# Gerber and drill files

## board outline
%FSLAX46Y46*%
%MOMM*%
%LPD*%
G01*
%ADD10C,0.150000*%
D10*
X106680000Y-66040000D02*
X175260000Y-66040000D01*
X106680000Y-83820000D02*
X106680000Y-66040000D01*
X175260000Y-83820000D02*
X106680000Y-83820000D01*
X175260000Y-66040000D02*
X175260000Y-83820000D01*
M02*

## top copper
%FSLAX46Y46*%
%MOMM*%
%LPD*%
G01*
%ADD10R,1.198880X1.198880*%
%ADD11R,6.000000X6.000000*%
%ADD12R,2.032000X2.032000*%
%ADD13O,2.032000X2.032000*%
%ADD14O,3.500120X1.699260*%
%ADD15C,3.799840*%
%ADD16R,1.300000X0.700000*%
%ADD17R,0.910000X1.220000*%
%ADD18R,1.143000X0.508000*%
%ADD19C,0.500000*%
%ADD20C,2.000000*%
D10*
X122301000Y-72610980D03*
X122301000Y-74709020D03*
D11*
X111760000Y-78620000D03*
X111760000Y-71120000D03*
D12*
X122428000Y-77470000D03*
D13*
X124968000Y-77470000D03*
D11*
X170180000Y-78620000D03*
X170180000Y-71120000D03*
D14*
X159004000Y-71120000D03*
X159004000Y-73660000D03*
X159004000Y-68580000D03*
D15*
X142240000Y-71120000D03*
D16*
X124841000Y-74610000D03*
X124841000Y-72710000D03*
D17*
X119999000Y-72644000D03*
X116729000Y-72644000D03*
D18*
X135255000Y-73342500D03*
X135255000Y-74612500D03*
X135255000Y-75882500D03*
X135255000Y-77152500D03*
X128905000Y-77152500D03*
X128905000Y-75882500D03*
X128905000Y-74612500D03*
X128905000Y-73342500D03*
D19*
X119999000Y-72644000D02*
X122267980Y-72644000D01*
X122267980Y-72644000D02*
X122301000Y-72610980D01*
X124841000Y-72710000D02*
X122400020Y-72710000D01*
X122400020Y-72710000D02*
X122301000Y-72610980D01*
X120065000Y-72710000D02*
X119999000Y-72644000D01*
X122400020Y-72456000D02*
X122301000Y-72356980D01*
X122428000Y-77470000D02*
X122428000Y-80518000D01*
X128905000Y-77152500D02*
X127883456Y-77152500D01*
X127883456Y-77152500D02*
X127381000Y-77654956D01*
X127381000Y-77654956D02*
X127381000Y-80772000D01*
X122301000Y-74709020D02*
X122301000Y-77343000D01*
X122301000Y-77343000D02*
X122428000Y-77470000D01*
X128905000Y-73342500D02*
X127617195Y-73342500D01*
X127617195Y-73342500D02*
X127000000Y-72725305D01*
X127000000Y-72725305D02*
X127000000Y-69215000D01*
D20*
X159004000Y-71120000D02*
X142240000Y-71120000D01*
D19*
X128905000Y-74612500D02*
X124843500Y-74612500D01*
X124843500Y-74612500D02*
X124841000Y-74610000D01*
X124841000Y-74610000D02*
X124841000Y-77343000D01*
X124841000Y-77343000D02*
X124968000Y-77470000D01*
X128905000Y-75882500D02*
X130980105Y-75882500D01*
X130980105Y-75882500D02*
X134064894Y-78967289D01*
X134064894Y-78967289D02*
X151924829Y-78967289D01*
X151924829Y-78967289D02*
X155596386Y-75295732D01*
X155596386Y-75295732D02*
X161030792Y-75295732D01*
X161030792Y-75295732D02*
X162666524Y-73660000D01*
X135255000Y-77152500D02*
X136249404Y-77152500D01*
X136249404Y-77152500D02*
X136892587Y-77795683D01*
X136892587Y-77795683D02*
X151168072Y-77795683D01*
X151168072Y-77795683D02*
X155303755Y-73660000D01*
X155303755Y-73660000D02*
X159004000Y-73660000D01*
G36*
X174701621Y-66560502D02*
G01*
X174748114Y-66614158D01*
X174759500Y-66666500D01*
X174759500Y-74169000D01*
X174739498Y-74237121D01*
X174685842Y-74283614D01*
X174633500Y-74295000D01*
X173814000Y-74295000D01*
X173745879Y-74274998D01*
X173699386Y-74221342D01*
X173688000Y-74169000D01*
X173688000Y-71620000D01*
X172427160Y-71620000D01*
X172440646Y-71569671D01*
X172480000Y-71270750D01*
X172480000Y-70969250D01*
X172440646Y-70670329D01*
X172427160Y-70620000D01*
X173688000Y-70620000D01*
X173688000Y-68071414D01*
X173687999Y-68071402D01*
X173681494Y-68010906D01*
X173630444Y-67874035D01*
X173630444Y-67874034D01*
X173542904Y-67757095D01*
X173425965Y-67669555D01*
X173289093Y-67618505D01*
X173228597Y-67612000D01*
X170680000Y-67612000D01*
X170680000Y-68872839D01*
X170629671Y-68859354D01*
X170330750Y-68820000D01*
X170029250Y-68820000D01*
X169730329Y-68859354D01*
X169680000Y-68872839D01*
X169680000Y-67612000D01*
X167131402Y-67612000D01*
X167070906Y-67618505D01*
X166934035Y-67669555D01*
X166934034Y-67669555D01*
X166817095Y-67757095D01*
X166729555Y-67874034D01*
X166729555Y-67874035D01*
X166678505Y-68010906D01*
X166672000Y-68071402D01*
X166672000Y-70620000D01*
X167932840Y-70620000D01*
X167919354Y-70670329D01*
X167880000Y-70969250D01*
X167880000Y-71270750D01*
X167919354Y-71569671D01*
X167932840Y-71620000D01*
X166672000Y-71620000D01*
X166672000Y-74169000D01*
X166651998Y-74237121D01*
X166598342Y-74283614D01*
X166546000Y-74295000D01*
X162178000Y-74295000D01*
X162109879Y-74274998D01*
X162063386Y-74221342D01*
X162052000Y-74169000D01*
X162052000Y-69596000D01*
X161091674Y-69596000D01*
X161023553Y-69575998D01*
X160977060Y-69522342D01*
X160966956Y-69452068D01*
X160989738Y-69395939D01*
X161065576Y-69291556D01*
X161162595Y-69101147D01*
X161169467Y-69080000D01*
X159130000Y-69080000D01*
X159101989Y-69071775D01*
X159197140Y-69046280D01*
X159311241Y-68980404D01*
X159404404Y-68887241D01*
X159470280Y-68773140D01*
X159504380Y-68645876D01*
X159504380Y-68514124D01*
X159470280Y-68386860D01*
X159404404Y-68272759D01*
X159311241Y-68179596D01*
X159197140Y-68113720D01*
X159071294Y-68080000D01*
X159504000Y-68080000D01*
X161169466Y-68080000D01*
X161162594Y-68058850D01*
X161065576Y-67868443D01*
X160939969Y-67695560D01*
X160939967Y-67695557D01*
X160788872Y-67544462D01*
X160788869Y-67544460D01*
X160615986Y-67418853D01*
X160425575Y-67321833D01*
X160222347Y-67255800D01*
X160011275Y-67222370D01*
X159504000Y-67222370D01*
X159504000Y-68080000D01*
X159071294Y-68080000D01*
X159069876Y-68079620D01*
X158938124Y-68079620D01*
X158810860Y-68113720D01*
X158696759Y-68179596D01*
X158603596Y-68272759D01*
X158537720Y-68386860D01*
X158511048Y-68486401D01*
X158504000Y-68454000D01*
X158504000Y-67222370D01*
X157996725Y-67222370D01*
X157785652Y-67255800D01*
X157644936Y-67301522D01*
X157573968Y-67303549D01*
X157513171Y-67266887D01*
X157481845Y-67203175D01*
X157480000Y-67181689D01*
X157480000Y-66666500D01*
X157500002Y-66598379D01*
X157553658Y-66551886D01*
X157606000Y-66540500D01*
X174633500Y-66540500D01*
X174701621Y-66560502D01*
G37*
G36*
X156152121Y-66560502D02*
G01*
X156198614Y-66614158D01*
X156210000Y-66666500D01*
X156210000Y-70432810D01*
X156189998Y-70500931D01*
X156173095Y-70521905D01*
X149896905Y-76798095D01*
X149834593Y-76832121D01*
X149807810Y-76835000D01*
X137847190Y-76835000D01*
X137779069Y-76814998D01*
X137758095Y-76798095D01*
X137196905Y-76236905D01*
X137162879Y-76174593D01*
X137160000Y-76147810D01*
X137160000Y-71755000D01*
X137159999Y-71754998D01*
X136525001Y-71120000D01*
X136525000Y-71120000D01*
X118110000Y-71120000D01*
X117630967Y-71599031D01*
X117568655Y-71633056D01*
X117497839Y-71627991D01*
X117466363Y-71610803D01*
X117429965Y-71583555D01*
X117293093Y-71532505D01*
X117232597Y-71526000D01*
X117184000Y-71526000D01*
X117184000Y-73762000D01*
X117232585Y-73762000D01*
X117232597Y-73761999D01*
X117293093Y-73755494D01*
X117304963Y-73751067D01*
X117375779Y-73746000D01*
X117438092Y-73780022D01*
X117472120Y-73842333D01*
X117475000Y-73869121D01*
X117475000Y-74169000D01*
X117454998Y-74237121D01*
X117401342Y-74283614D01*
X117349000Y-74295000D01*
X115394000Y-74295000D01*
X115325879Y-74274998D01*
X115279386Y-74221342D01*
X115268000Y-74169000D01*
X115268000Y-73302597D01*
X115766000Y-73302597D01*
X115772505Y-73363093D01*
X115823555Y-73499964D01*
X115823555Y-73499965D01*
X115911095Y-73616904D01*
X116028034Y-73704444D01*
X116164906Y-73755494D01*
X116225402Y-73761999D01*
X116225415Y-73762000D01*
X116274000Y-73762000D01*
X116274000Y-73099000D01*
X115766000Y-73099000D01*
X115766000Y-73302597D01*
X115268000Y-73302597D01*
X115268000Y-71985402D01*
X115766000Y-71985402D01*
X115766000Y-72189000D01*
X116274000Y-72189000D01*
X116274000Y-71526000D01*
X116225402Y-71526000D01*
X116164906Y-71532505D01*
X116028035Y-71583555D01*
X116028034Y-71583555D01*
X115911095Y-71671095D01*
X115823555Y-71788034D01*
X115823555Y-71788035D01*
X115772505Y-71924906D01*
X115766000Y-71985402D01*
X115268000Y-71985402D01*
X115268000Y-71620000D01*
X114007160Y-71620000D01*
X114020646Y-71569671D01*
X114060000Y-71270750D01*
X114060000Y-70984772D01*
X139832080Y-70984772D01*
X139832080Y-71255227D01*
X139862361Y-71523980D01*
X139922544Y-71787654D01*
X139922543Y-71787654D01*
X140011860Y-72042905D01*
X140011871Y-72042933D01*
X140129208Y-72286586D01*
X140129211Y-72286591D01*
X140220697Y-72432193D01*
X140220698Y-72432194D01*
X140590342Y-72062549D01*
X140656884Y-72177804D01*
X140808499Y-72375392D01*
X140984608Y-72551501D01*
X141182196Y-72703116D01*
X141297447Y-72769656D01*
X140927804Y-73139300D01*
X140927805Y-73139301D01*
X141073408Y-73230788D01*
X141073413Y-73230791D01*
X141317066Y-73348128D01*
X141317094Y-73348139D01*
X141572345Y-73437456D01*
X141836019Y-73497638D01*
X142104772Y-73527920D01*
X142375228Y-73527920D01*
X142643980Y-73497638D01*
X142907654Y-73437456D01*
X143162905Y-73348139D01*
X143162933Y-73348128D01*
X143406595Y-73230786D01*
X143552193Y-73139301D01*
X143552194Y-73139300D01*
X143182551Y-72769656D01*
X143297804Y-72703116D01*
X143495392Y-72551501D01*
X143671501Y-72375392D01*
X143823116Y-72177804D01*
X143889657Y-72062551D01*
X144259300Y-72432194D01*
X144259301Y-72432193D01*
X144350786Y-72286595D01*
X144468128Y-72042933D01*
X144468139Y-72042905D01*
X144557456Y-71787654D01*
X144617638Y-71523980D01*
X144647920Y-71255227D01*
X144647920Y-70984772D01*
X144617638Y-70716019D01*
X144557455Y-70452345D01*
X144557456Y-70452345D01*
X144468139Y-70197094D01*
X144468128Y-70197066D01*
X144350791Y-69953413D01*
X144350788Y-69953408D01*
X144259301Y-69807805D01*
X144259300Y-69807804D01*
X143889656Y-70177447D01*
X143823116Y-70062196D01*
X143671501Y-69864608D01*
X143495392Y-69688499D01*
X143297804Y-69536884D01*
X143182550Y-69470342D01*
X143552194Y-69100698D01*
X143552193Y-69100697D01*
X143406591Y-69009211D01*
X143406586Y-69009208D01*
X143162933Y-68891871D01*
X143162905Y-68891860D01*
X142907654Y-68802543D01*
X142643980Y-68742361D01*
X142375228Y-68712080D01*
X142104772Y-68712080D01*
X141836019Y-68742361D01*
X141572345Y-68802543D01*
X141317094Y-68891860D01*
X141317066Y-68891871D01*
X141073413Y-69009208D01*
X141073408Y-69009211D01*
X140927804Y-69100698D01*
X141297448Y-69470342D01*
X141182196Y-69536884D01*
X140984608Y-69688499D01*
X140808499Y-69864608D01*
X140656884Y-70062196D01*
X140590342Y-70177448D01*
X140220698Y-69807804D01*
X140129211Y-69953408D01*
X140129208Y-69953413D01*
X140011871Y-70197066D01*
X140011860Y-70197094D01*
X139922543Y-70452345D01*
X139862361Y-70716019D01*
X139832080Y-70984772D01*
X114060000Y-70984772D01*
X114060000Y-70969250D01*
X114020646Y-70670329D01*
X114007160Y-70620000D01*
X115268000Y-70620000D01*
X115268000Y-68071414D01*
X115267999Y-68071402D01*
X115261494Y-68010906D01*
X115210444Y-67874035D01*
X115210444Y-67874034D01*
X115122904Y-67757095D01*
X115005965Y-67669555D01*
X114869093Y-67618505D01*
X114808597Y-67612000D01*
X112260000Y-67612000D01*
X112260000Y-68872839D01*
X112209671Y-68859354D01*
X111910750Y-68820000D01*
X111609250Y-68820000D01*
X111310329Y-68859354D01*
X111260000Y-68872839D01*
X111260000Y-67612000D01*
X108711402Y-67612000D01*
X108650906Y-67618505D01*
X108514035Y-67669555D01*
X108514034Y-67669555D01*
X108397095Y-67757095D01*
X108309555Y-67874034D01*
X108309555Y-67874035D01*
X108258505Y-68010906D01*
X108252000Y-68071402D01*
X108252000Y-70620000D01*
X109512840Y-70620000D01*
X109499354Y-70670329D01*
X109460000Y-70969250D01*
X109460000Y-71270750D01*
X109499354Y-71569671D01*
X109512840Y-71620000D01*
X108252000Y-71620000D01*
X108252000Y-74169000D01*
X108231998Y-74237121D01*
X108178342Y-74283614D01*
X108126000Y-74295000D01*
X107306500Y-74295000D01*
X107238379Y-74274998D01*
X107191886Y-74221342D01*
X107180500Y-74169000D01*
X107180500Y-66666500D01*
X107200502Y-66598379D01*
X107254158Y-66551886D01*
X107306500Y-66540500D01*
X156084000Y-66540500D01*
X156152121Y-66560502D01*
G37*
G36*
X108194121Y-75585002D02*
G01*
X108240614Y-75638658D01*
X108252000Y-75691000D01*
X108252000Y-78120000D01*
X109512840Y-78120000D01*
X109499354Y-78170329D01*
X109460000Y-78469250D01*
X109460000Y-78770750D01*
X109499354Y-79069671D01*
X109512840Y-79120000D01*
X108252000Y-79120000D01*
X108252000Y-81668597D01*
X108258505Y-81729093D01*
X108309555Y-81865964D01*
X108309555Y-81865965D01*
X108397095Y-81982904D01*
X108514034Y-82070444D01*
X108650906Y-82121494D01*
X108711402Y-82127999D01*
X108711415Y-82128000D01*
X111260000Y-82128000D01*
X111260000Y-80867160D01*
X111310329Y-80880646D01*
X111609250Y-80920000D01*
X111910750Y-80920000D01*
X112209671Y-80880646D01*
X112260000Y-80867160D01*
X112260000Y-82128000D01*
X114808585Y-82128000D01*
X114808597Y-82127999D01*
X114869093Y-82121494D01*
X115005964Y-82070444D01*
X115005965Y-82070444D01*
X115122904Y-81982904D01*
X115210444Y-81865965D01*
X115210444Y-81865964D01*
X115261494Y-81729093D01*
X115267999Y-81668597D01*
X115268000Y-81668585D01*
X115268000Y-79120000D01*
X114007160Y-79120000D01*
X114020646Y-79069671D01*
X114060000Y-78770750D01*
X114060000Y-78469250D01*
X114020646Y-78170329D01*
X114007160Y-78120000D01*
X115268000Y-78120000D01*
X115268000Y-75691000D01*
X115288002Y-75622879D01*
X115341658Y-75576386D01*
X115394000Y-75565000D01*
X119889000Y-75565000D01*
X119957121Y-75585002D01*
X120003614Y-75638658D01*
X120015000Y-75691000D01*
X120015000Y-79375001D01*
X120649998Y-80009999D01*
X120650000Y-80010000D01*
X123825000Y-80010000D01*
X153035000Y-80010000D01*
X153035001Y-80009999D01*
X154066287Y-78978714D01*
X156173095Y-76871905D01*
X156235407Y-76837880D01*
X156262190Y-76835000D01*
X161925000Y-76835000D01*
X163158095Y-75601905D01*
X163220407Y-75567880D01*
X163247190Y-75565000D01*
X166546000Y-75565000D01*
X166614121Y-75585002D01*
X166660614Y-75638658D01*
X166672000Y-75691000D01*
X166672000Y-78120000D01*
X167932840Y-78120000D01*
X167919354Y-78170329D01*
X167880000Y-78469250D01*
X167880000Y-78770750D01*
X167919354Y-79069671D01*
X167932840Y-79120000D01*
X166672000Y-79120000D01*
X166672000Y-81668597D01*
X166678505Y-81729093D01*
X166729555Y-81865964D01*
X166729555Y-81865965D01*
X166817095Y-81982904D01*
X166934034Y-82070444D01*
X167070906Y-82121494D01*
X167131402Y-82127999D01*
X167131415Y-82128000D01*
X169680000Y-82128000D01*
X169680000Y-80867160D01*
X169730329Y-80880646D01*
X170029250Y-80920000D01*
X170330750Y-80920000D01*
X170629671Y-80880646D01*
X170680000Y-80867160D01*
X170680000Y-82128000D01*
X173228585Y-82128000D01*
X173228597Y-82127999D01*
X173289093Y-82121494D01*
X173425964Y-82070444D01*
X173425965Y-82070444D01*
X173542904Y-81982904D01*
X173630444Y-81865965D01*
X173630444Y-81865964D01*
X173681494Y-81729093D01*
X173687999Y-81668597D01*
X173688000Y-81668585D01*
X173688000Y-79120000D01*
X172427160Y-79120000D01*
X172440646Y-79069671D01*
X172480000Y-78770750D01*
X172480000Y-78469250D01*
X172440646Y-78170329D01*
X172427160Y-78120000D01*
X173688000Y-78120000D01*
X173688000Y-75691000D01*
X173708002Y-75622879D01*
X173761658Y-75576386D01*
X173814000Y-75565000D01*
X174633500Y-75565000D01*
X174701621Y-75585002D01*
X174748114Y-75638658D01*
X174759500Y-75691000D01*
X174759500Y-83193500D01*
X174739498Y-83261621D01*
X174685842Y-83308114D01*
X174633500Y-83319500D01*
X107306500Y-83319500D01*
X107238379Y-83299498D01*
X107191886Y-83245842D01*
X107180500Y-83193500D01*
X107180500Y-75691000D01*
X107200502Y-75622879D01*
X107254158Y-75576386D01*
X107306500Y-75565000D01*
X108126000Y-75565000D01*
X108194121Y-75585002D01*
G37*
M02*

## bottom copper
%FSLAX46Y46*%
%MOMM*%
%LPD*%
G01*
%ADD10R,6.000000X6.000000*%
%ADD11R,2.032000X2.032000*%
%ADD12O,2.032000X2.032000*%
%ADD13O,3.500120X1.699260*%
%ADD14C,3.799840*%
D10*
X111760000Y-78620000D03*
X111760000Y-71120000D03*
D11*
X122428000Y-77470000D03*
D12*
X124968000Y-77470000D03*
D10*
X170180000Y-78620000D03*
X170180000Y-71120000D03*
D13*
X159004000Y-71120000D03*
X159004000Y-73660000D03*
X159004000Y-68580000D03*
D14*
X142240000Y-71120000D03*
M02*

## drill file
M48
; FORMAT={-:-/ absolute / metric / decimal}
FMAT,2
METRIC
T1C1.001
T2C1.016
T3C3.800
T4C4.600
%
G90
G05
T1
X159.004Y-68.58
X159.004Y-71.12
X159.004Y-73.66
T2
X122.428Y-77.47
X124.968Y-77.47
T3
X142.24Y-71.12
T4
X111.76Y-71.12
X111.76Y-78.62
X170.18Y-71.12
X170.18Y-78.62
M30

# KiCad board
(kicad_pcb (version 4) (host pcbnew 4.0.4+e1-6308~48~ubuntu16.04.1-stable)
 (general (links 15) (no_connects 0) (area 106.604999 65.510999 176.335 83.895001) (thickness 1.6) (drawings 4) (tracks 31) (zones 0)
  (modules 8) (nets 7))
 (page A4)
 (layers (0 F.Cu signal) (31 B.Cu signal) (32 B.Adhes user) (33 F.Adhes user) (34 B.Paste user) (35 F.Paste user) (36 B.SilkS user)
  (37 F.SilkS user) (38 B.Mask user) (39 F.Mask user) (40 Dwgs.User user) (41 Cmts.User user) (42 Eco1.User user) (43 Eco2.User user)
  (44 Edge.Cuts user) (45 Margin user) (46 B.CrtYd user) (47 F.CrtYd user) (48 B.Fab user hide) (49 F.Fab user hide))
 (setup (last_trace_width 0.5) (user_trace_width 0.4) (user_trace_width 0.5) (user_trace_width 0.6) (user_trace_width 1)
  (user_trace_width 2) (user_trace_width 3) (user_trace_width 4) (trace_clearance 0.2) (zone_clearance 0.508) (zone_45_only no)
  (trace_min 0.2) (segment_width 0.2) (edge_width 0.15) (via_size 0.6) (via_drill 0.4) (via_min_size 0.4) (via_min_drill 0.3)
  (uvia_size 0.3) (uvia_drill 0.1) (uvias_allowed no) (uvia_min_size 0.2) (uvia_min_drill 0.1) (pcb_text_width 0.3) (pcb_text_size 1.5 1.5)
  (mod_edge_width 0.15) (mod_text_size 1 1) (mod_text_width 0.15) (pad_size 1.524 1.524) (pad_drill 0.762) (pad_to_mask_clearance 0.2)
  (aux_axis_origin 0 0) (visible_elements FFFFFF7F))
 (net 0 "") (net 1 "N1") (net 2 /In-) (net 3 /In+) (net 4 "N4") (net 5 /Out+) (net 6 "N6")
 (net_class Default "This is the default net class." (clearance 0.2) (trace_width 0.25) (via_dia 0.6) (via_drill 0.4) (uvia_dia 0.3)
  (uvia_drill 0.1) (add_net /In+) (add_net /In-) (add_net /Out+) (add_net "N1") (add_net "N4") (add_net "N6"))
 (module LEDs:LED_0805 (layer F.Cu) (at 122.301 73.66 90)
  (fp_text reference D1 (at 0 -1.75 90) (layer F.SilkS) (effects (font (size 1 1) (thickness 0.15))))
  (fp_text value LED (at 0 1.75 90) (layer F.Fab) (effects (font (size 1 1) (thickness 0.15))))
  (pad 2 smd rect (at 1.04902 0 270) (size 1.19888 1.19888) (layers F.Cu F.Paste F.Mask) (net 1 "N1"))
  (pad 1 smd rect (at -1.04902 0 270) (size 1.19888 1.19888) (layers F.Cu F.Paste F.Mask) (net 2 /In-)))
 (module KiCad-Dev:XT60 (layer B.Cu) (at 111.76 78.62 90)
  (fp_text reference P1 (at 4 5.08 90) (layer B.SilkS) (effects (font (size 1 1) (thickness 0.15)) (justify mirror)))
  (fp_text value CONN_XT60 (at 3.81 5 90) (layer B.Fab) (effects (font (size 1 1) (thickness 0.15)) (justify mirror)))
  (pad 1 thru_hole rect (at 0 0 90) (size 6 6) (drill 4.6) (layers *.Cu *.Mask) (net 2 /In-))
  (pad 2 thru_hole rect (at 7.5 0 90) (size 6 6) (drill 4.6) (layers *.Cu *.Mask) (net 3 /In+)))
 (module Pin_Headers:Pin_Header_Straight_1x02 (layer B.Cu) (at 122.428 77.47 270)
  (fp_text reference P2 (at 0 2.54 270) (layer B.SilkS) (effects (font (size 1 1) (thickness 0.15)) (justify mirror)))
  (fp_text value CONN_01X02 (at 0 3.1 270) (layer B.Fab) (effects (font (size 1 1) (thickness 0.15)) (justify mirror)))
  (pad 1 thru_hole rect (at 0 0 270) (size 2.032 2.032) (drill 1.016) (layers *.Cu *.Mask) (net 2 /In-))
  (pad 2 thru_hole oval (at 0 -2.54 270) (size 2.032 2.032) (drill 1.016) (layers *.Cu *.Mask) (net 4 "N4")))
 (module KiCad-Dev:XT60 (layer B.Cu) (at 170.18 78.62 90)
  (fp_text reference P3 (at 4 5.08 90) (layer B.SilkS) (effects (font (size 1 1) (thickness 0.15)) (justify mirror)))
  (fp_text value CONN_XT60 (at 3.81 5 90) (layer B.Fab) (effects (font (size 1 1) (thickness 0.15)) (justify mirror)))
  (pad 1 thru_hole rect (at 0 0 90) (size 6 6) (drill 4.6) (layers *.Cu *.Mask) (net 2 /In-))
  (pad 2 thru_hole rect (at 7.5 0 90) (size 6 6) (drill 4.6) (layers *.Cu *.Mask) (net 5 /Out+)))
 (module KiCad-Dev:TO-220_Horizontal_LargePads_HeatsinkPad (layer F.Cu) (at 159.004 71.12 90)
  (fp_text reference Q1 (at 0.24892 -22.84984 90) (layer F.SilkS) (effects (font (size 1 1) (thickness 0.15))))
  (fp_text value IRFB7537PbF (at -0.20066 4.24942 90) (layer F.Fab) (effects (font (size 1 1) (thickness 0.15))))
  (pad 2 thru_hole oval (at 0 0 180) (size 3.50012 1.69926) (drill 1.00076) (layers *.Cu *.Mask F.SilkS) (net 3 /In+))
  (pad 1 thru_hole oval (at -2.54 0 180) (size 3.50012 1.69926) (drill 1.00076) (layers *.Cu *.Mask F.SilkS) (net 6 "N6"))
  (pad 3 thru_hole oval (at 2.54 0 180) (size 3.50012 1.69926) (drill 1.00076) (layers *.Cu *.Mask F.SilkS) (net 5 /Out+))
  (pad 2 thru_hole circle (at 0 -16.764 180) (size 3.79984 3.79984) (drill 3.79984) (layers *.Cu *.Mask) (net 3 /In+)))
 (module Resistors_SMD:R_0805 (layer F.Cu) (at 124.841 73.66 90)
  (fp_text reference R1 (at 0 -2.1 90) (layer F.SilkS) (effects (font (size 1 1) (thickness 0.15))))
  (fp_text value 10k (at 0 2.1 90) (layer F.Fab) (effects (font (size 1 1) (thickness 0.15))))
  (pad 1 smd rect (at -0.95 0 90) (size 0.7 1.3) (layers F.Cu F.Paste F.Mask) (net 4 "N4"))
  (pad 2 smd rect (at 0.95 0 90) (size 0.7 1.3) (layers F.Cu F.Paste F.Mask) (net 1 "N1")))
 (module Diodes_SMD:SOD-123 (layer F.Cu) (at 118.364 72.644 180)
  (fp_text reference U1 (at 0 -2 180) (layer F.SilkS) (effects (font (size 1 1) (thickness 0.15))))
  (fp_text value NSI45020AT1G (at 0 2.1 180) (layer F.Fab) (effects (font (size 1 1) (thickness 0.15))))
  (pad 1 smd rect (at -1.635 0 180) (size 0.91 1.22) (layers F.Cu F.Paste F.Mask) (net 1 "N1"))
  (pad 2 smd rect (at 1.635 0 180) (size 0.91 1.22) (layers F.Cu F.Paste F.Mask) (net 3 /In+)))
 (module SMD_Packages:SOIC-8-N (layer F.Cu) (at 132.08 75.2475 270)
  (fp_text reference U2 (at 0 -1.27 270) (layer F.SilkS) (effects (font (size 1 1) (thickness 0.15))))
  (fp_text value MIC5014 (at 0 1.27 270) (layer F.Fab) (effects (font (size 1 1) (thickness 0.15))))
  (pad 8 smd rect (at -1.905 -3.175 270) (size 0.508 1.143) (layers F.Cu F.Paste F.Mask))
  (pad 7 smd rect (at -0.635 -3.175 270) (size 0.508 1.143) (layers F.Cu F.Paste F.Mask))
  (pad 6 smd rect (at 0.635 -3.175 270) (size 0.508 1.143) (layers F.Cu F.Paste F.Mask))
  (pad 5 smd rect (at 1.905 -3.175 270) (size 0.508 1.143) (layers F.Cu F.Paste F.Mask) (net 6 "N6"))
  (pad 4 smd rect (at 1.905 3.175 270) (size 0.508 1.143) (layers F.Cu F.Paste F.Mask) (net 2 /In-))
  (pad 3 smd rect (at 0.635 3.175 270) (size 0.508 1.143) (layers F.Cu F.Paste F.Mask) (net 5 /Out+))
  (pad 2 smd rect (at -0.635 3.175 270) (size 0.508 1.143) (layers F.Cu F.Paste F.Mask) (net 4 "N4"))
  (pad 1 smd rect (at -1.905 3.175 270) (size 0.508 1.143) (layers F.Cu F.Paste F.Mask) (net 3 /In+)))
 (gr_line (start 106.68 66.04) (end 175.26 66.04) (layer Edge.Cuts) (width 0.15))
 (gr_line (start 106.68 83.82) (end 106.68 66.04) (layer Edge.Cuts) (width 0.15))
 (gr_line (start 175.26 83.82) (end 106.68 83.82) (layer Edge.Cuts) (width 0.15))
 (gr_line (start 175.26 66.04) (end 175.26 83.82) (layer Edge.Cuts) (width 0.15))
 (segment (start 119.999 72.644) (end 122.26798 72.644) (width 0.5) (layer F.Cu) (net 1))
 (segment (start 122.26798 72.644) (end 122.301 72.61098) (width 0.5) (layer F.Cu) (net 1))
 (segment (start 124.841 72.71) (end 122.40002 72.71) (width 0.5) (layer F.Cu) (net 1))
 (segment (start 122.40002 72.71) (end 122.301 72.61098) (width 0.5) (layer F.Cu) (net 1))
 (segment (start 120.065 72.71) (end 119.999 72.644) (width 0.5) (layer F.Cu) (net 1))
 (segment (start 122.40002 72.456) (end 122.301 72.35698) (width 0.5) (layer F.Cu) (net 1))
 (segment (start 122.428 77.47) (end 122.428 80.518) (width 0.5) (layer F.Cu) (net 2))
 (segment (start 128.905 77.1525) (end 127.883456 77.1525) (width 0.5) (layer F.Cu) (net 2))
 (segment (start 127.883456 77.1525) (end 127.381 77.654956) (width 0.5) (layer F.Cu) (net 2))
 (segment (start 127.381 77.654956) (end 127.381 80.772) (width 0.5) (layer F.Cu) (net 2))
 (segment (start 122.301 74.70902) (end 122.301 77.343) (width 0.5) (layer F.Cu) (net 2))
 (segment (start 122.301 77.343) (end 122.428 77.47) (width 0.5) (layer F.Cu) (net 2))
 (segment (start 128.905 73.3425) (end 127.617195 73.3425) (width 0.5) (layer F.Cu) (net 3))
 (segment (start 127.617195 73.3425) (end 127 72.725305) (width 0.5) (layer F.Cu) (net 3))
 (segment (start 127 72.725305) (end 127 69.215) (width 0.5) (layer F.Cu) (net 3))
 (segment (start 159.004 71.12) (end 142.24 71.12) (width 2) (layer F.Cu) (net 3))
 (segment (start 128.905 74.6125) (end 124.8435 74.6125) (width 0.5) (layer F.Cu) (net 4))
 (segment (start 124.8435 74.6125) (end 124.841 74.61) (width 0.5) (layer F.Cu) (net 4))
 (segment (start 124.841 74.61) (end 124.841 77.343) (width 0.5) (layer F.Cu) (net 4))
 (segment (start 124.841 77.343) (end 124.968 77.47) (width 0.5) (layer F.Cu) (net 4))
 (segment (start 128.905 75.8825) (end 130.980105 75.8825) (width 0.5) (layer F.Cu) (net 5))
 (segment (start 130.980105 75.8825) (end 134.064894 78.967289) (width 0.5) (layer F.Cu) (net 5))
 (segment (start 134.064894 78.967289) (end 151.924829 78.967289) (width 0.5) (layer F.Cu) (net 5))
 (segment (start 151.924829 78.967289) (end 155.596386 75.295732) (width 0.5) (layer F.Cu) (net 5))
 (segment (start 155.596386 75.295732) (end 161.030792 75.295732) (width 0.5) (layer F.Cu) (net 5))
 (segment (start 161.030792 75.295732) (end 162.666524 73.66) (width 0.5) (layer F.Cu) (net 5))
 (segment (start 135.255 77.1525) (end 136.249404 77.1525) (width 0.5) (layer F.Cu) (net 6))
 (segment (start 136.249404 77.1525) (end 136.892587 77.795683) (width 0.5) (layer F.Cu) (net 6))
 (segment (start 136.892587 77.795683) (end 151.168072 77.795683) (width 0.5) (layer F.Cu) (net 6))
 (segment (start 151.168072 77.795683) (end 155.303755 73.66) (width 0.5) (layer F.Cu) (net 6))
 (segment (start 155.303755 73.66) (end 159.004 73.66) (width 0.5) (layer F.Cu) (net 6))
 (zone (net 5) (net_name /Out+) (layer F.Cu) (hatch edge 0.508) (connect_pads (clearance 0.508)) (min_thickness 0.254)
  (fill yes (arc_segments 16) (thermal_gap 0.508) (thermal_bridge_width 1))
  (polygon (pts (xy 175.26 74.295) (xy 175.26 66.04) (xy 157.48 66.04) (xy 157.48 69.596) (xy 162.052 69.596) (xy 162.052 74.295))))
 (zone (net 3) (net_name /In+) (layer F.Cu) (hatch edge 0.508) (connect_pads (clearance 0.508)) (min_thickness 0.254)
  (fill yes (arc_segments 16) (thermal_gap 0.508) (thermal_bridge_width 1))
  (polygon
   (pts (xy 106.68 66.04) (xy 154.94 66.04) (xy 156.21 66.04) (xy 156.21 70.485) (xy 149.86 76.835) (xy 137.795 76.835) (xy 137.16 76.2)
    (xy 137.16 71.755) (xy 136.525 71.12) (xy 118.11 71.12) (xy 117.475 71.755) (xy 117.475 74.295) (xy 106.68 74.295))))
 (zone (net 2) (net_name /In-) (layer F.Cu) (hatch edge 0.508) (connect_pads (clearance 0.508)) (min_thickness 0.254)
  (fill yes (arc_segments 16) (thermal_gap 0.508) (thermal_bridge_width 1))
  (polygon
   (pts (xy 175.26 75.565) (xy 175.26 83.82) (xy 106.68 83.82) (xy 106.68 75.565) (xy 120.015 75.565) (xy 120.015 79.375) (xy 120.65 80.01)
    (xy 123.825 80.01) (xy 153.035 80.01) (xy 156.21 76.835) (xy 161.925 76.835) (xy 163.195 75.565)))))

